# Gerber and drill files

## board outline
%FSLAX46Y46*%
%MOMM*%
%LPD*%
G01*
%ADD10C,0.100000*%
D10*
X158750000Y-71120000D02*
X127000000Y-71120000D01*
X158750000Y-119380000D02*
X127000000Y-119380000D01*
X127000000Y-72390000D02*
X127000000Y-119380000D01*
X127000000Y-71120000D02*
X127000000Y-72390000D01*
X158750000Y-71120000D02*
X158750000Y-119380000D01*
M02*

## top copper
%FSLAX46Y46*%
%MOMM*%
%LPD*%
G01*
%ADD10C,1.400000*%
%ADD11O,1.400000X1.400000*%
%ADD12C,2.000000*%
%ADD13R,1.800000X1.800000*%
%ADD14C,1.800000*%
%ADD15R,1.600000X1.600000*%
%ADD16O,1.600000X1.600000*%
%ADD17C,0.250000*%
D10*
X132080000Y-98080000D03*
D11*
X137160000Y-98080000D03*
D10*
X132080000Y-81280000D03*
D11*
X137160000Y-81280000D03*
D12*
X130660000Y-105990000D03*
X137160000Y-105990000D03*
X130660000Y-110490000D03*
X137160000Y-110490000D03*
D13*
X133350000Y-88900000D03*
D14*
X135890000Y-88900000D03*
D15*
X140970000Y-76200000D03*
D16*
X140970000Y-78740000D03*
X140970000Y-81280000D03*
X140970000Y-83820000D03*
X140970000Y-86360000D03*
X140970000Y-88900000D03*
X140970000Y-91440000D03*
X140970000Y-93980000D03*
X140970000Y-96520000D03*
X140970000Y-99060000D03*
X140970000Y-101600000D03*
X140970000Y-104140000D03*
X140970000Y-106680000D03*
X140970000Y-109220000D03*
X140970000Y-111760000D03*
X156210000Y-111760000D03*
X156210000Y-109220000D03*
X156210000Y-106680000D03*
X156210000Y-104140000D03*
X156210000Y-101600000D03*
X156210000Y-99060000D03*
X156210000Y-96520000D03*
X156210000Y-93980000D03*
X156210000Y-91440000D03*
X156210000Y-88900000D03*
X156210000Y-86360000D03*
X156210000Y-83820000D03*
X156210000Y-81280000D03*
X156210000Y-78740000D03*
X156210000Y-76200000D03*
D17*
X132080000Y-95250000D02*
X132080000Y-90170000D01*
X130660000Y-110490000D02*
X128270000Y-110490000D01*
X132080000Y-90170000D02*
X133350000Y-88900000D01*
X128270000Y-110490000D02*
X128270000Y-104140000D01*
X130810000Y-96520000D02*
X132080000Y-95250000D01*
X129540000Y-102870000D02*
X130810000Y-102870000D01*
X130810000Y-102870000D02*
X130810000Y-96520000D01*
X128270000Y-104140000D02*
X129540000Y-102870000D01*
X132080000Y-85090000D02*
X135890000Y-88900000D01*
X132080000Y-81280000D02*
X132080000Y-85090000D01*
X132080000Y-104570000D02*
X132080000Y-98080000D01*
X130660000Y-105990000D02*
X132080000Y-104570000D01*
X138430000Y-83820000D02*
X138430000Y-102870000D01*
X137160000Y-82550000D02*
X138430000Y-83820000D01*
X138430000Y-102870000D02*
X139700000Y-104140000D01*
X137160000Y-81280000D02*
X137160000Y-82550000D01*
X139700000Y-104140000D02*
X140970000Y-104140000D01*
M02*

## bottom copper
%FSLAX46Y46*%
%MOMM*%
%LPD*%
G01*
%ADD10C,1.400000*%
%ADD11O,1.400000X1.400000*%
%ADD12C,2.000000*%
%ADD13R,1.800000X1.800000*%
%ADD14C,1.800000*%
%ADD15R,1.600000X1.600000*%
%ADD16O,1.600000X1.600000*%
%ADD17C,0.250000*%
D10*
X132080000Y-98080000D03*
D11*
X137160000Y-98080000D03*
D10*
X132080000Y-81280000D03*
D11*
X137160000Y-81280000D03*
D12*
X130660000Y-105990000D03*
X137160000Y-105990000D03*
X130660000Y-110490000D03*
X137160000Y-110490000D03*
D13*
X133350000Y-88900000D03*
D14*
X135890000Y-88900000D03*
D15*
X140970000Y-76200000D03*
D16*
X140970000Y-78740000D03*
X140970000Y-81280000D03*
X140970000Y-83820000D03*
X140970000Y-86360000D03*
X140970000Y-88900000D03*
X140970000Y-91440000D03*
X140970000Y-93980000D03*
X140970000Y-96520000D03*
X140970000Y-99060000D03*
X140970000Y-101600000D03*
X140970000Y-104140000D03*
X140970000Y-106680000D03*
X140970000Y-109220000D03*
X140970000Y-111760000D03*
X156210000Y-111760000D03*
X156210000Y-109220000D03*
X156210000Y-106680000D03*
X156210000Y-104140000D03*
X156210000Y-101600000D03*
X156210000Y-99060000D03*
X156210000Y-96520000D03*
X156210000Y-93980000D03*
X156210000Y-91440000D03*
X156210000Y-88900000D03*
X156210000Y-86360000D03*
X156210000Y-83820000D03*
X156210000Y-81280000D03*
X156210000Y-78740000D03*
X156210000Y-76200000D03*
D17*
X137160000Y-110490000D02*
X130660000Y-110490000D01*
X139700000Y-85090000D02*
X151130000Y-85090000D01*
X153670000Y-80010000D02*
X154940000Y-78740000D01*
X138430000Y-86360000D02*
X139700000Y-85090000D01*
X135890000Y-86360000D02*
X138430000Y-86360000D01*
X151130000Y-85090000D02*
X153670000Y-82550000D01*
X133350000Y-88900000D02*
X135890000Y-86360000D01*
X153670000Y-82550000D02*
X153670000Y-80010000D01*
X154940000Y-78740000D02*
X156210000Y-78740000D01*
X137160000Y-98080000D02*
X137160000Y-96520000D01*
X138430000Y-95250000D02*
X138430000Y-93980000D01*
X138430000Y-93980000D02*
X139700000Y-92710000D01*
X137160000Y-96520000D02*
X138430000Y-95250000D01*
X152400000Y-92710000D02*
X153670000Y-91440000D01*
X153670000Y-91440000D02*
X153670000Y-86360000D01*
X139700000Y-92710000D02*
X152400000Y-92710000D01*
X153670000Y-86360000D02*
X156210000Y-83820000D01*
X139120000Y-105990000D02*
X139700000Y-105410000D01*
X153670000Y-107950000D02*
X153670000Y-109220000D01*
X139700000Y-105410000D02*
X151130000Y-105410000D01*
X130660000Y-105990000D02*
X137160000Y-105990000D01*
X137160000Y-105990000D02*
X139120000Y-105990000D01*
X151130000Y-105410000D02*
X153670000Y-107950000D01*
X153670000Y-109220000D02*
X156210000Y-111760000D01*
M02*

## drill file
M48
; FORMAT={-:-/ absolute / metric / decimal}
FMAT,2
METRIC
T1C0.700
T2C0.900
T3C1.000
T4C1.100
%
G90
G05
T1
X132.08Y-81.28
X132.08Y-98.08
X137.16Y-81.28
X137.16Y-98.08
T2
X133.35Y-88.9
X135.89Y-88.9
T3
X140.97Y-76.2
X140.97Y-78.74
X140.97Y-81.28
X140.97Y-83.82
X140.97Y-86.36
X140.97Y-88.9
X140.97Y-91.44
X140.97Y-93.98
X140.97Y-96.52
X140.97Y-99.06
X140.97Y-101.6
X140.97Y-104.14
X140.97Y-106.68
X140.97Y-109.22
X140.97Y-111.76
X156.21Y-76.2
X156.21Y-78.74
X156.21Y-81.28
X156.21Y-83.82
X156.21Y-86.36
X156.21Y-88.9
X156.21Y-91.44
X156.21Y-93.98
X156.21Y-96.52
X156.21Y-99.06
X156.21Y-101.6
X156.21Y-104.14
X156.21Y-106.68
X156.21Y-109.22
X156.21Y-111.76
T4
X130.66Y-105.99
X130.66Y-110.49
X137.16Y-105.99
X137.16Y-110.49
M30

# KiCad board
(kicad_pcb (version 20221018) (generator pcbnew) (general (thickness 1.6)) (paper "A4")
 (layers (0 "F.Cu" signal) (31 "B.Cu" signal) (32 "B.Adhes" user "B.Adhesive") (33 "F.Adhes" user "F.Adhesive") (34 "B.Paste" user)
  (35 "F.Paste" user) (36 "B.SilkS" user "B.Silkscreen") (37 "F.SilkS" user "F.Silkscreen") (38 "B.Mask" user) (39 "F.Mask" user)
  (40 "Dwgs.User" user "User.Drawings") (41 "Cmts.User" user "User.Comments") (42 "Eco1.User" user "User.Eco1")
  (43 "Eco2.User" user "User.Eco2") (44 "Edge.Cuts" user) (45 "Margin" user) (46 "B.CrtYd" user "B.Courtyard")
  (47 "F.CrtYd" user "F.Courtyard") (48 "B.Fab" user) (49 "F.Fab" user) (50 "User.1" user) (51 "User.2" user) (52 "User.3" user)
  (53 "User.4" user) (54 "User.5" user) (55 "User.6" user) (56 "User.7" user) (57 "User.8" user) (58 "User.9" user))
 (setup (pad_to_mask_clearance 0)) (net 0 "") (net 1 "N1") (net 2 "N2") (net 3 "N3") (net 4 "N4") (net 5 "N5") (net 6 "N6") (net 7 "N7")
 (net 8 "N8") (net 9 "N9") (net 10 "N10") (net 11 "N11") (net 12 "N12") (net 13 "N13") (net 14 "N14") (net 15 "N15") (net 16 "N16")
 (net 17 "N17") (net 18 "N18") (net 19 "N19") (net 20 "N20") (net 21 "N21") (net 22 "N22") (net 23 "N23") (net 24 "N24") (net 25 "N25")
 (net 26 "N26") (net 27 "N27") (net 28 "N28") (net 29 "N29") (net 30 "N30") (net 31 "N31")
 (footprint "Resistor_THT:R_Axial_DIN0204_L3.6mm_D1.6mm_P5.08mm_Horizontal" (layer "F.Cu") (at 132.08 98.08)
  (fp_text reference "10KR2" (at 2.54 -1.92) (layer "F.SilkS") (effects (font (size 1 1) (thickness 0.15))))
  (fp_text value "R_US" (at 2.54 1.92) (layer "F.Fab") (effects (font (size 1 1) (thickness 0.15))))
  (pad "1" thru_hole circle (at 0 0) (size 1.4 1.4) (drill 0.7) (layers "*.Cu" "*.Mask") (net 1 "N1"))
  (pad "2" thru_hole oval (at 5.08 0) (size 1.4 1.4) (drill 0.7) (layers "*.Cu" "*.Mask") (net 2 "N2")))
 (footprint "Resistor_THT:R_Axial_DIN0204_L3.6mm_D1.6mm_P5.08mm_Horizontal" (layer "F.Cu") (at 132.08 81.28)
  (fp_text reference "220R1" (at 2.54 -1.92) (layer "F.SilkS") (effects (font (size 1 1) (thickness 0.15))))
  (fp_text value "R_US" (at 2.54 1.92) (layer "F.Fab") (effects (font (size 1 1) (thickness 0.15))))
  (pad "1" thru_hole circle (at 0 0) (size 1.4 1.4) (drill 0.7) (layers "*.Cu" "*.Mask") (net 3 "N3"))
  (pad "2" thru_hole oval (at 5.08 0) (size 1.4 1.4) (drill 0.7) (layers "*.Cu" "*.Mask") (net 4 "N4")))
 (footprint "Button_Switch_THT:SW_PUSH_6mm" (layer "F.Cu") (at 130.66 105.99)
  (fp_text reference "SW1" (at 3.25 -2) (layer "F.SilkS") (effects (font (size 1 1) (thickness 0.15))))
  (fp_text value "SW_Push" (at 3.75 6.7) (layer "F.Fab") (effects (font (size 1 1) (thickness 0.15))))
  (pad "1" thru_hole circle (at 0 0 90) (size 2 2) (drill 1.1) (layers "*.Cu" "*.Mask") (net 1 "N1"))
  (pad "1" thru_hole circle (at 6.5 0 90) (size 2 2) (drill 1.1) (layers "*.Cu" "*.Mask") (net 1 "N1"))
  (pad "2" thru_hole circle (at 0 4.5 90) (size 2 2) (drill 1.1) (layers "*.Cu" "*.Mask") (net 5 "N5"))
  (pad "2" thru_hole circle (at 6.5 4.5 90) (size 2 2) (drill 1.1) (layers "*.Cu" "*.Mask") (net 5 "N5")))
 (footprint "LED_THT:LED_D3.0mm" (layer "F.Cu") (at 133.35 88.9)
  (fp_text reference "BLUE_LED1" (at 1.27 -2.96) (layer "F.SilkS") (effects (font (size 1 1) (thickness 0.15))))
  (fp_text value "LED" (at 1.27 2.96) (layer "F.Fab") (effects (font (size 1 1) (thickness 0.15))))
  (pad "1" thru_hole rect (at 0 0) (size 1.8 1.8) (drill 0.9) (layers "*.Cu" "*.Mask") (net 5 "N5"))
  (pad "2" thru_hole circle (at 2.54 0) (size 1.8 1.8) (drill 0.9) (layers "*.Cu" "*.Mask") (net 3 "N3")))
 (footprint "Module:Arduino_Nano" (layer "F.Cu") (at 140.97 76.2)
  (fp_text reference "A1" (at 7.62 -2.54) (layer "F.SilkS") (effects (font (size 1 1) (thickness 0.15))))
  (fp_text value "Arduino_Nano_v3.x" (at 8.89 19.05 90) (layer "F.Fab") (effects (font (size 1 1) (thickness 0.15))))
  (pad "1" thru_hole rect (at 0 0) (size 1.6 1.6) (drill 1) (layers "*.Cu" "*.Mask") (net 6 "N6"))
  (pad "2" thru_hole oval (at 0 2.54) (size 1.6 1.6) (drill 1) (layers "*.Cu" "*.Mask") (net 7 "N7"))
  (pad "3" thru_hole oval (at 0 5.08) (size 1.6 1.6) (drill 1) (layers "*.Cu" "*.Mask") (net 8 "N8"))
  (pad "4" thru_hole oval (at 0 7.62) (size 1.6 1.6) (drill 1) (layers "*.Cu" "*.Mask") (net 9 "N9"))
  (pad "5" thru_hole oval (at 0 10.16) (size 1.6 1.6) (drill 1) (layers "*.Cu" "*.Mask") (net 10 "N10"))
  (pad "6" thru_hole oval (at 0 12.7) (size 1.6 1.6) (drill 1) (layers "*.Cu" "*.Mask") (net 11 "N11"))
  (pad "7" thru_hole oval (at 0 15.24) (size 1.6 1.6) (drill 1) (layers "*.Cu" "*.Mask") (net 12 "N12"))
  (pad "8" thru_hole oval (at 0 17.78) (size 1.6 1.6) (drill 1) (layers "*.Cu" "*.Mask") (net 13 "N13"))
  (pad "9" thru_hole oval (at 0 20.32) (size 1.6 1.6) (drill 1) (layers "*.Cu" "*.Mask") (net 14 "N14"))
  (pad "10" thru_hole oval (at 0 22.86) (size 1.6 1.6) (drill 1) (layers "*.Cu" "*.Mask") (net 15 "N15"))
  (pad "11" thru_hole oval (at 0 25.4) (size 1.6 1.6) (drill 1) (layers "*.Cu" "*.Mask") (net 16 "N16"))
  (pad "12" thru_hole oval (at 0 27.94) (size 1.6 1.6) (drill 1) (layers "*.Cu" "*.Mask") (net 4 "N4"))
  (pad "13" thru_hole oval (at 0 30.48) (size 1.6 1.6) (drill 1) (layers "*.Cu" "*.Mask") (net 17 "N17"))
  (pad "14" thru_hole oval (at 0 33.02) (size 1.6 1.6) (drill 1) (layers "*.Cu" "*.Mask") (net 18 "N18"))
  (pad "15" thru_hole oval (at 0 35.56) (size 1.6 1.6) (drill 1) (layers "*.Cu" "*.Mask") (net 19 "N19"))
  (pad "16" thru_hole oval (at 15.24 35.56) (size 1.6 1.6) (drill 1) (layers "*.Cu" "*.Mask") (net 1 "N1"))
  (pad "17" thru_hole oval (at 15.24 33.02) (size 1.6 1.6) (drill 1) (layers "*.Cu" "*.Mask") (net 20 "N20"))
  (pad "18" thru_hole oval (at 15.24 30.48) (size 1.6 1.6) (drill 1) (layers "*.Cu" "*.Mask") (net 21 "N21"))
  (pad "19" thru_hole oval (at 15.24 27.94) (size 1.6 1.6) (drill 1) (layers "*.Cu" "*.Mask") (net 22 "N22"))
  (pad "20" thru_hole oval (at 15.24 25.4) (size 1.6 1.6) (drill 1) (layers "*.Cu" "*.Mask") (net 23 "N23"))
  (pad "21" thru_hole oval (at 15.24 22.86) (size 1.6 1.6) (drill 1) (layers "*.Cu" "*.Mask") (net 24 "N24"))
  (pad "22" thru_hole oval (at 15.24 20.32) (size 1.6 1.6) (drill 1) (layers "*.Cu" "*.Mask") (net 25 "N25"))
  (pad "23" thru_hole oval (at 15.24 17.78) (size 1.6 1.6) (drill 1) (layers "*.Cu" "*.Mask") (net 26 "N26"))
  (pad "24" thru_hole oval (at 15.24 15.24) (size 1.6 1.6) (drill 1) (layers "*.Cu" "*.Mask") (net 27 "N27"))
  (pad "25" thru_hole oval (at 15.24 12.7) (size 1.6 1.6) (drill 1) (layers "*.Cu" "*.Mask") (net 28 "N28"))
  (pad "26" thru_hole oval (at 15.24 10.16) (size 1.6 1.6) (drill 1) (layers "*.Cu" "*.Mask") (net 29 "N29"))
  (pad "27" thru_hole oval (at 15.24 7.62) (size 1.6 1.6) (drill 1) (layers "*.Cu" "*.Mask") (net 2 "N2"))
  (pad "28" thru_hole oval (at 15.24 5.08) (size 1.6 1.6) (drill 1) (layers "*.Cu" "*.Mask") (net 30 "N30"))
  (pad "29" thru_hole oval (at 15.24 2.54) (size 1.6 1.6) (drill 1) (layers "*.Cu" "*.Mask") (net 5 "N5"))
  (pad "30" thru_hole oval (at 15.24 0) (size 1.6 1.6) (drill 1) (layers "*.Cu" "*.Mask") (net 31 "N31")))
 (gr_line (start 158.75 71.12) (end 127 71.12) (stroke (width 0.1) (type default)) (layer "Edge.Cuts"))
 (gr_line (start 158.75 119.38) (end 127 119.38) (stroke (width 0.1) (type default)) (layer "Edge.Cuts"))
 (gr_line (start 127 72.39) (end 127 119.38) (stroke (width 0.1) (type default)) (layer "Edge.Cuts"))
 (gr_line (start 127 71.12) (end 127 72.39) (stroke (width 0.1) (type default)) (layer "Edge.Cuts"))
 (gr_line (start 158.75 71.12) (end 158.75 119.38) (stroke (width 0.1) (type default)) (layer "Edge.Cuts"))
 (segment (start 132.08 95.25) (end 132.08 90.17) (width 0.25) (layer "F.Cu") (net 5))
 (segment (start 130.66 110.49) (end 128.27 110.49) (width 0.25) (layer "F.Cu") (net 5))
 (segment (start 132.08 90.17) (end 133.35 88.9) (width 0.25) (layer "F.Cu") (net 5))
 (segment (start 128.27 110.49) (end 128.27 104.14) (width 0.25) (layer "F.Cu") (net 5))
 (segment (start 130.81 96.52) (end 132.08 95.25) (width 0.25) (layer "F.Cu") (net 5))
 (segment (start 129.54 102.87) (end 130.81 102.87) (width 0.25) (layer "F.Cu") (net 5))
 (segment (start 130.81 102.87) (end 130.81 96.52) (width 0.25) (layer "F.Cu") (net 5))
 (segment (start 128.27 104.14) (end 129.54 102.87) (width 0.25) (layer "F.Cu") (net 5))
 (segment (start 137.16 110.49) (end 130.66 110.49) (width 0.25) (layer "B.Cu") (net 5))
 (segment (start 139.7 85.09) (end 151.13 85.09) (width 0.25) (layer "B.Cu") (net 5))
 (segment (start 153.67 80.01) (end 154.94 78.74) (width 0.25) (layer "B.Cu") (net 5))
 (segment (start 138.43 86.36) (end 139.7 85.09) (width 0.25) (layer "B.Cu") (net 5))
 (segment (start 135.89 86.36) (end 138.43 86.36) (width 0.25) (layer "B.Cu") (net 5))
 (segment (start 151.13 85.09) (end 153.67 82.55) (width 0.25) (layer "B.Cu") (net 5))
 (segment (start 133.35 88.9) (end 135.89 86.36) (width 0.25) (layer "B.Cu") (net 5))
 (segment (start 153.67 82.55) (end 153.67 80.01) (width 0.25) (layer "B.Cu") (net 5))
 (segment (start 154.94 78.74) (end 156.21 78.74) (width 0.25) (layer "B.Cu") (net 5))
 (segment (start 137.16 98.08) (end 137.16 96.52) (width 0.25) (layer "B.Cu") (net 2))
 (segment (start 138.43 95.25) (end 138.43 93.98) (width 0.25) (layer "B.Cu") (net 2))
 (segment (start 138.43 93.98) (end 139.7 92.71) (width 0.25) (layer "B.Cu") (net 2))
 (segment (start 137.16 96.52) (end 138.43 95.25) (width 0.25) (layer "B.Cu") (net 2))
 (segment (start 152.4 92.71) (end 153.67 91.44) (width 0.25) (layer "B.Cu") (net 2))
 (segment (start 153.67 91.44) (end 153.67 86.36) (width 0.25) (layer "B.Cu") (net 2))
 (segment (start 139.7 92.71) (end 152.4 92.71) (width 0.25) (layer "B.Cu") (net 2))
 (segment (start 153.67 86.36) (end 156.21 83.82) (width 0.25) (layer "B.Cu") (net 2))
 (segment (start 132.08 85.09) (end 135.89 88.9) (width 0.25) (layer "F.Cu") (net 3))
 (segment (start 132.08 81.28) (end 132.08 85.09) (width 0.25) (layer "F.Cu") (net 3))
 (segment (start 132.08 104.57) (end 132.08 98.08) (width 0.25) (layer "F.Cu") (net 1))
 (segment (start 130.66 105.99) (end 132.08 104.57) (width 0.25) (layer "F.Cu") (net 1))
 (segment (start 139.12 105.99) (end 139.7 105.41) (width 0.25) (layer "B.Cu") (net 1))
 (segment (start 153.67 107.95) (end 153.67 109.22) (width 0.25) (layer "B.Cu") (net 1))
 (segment (start 139.7 105.41) (end 151.13 105.41) (width 0.25) (layer "B.Cu") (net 1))
 (segment (start 130.66 105.99) (end 137.16 105.99) (width 0.25) (layer "B.Cu") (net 1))
 (segment (start 137.16 105.99) (end 139.12 105.99) (width 0.25) (layer "B.Cu") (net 1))
 (segment (start 151.13 105.41) (end 153.67 107.95) (width 0.25) (layer "B.Cu") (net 1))
 (segment (start 153.67 109.22) (end 156.21 111.76) (width 0.25) (layer "B.Cu") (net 1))
 (segment (start 138.43 83.82) (end 138.43 102.87) (width 0.25) (layer "F.Cu") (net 4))
 (segment (start 137.16 82.55) (end 138.43 83.82) (width 0.25) (layer "F.Cu") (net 4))
 (segment (start 138.43 102.87) (end 139.7 104.14) (width 0.25) (layer "F.Cu") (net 4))
 (segment (start 137.16 81.28) (end 137.16 82.55) (width 0.25) (layer "F.Cu") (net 4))
 (segment (start 139.7 104.14) (end 140.97 104.14) (width 0.25) (layer "F.Cu") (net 4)))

